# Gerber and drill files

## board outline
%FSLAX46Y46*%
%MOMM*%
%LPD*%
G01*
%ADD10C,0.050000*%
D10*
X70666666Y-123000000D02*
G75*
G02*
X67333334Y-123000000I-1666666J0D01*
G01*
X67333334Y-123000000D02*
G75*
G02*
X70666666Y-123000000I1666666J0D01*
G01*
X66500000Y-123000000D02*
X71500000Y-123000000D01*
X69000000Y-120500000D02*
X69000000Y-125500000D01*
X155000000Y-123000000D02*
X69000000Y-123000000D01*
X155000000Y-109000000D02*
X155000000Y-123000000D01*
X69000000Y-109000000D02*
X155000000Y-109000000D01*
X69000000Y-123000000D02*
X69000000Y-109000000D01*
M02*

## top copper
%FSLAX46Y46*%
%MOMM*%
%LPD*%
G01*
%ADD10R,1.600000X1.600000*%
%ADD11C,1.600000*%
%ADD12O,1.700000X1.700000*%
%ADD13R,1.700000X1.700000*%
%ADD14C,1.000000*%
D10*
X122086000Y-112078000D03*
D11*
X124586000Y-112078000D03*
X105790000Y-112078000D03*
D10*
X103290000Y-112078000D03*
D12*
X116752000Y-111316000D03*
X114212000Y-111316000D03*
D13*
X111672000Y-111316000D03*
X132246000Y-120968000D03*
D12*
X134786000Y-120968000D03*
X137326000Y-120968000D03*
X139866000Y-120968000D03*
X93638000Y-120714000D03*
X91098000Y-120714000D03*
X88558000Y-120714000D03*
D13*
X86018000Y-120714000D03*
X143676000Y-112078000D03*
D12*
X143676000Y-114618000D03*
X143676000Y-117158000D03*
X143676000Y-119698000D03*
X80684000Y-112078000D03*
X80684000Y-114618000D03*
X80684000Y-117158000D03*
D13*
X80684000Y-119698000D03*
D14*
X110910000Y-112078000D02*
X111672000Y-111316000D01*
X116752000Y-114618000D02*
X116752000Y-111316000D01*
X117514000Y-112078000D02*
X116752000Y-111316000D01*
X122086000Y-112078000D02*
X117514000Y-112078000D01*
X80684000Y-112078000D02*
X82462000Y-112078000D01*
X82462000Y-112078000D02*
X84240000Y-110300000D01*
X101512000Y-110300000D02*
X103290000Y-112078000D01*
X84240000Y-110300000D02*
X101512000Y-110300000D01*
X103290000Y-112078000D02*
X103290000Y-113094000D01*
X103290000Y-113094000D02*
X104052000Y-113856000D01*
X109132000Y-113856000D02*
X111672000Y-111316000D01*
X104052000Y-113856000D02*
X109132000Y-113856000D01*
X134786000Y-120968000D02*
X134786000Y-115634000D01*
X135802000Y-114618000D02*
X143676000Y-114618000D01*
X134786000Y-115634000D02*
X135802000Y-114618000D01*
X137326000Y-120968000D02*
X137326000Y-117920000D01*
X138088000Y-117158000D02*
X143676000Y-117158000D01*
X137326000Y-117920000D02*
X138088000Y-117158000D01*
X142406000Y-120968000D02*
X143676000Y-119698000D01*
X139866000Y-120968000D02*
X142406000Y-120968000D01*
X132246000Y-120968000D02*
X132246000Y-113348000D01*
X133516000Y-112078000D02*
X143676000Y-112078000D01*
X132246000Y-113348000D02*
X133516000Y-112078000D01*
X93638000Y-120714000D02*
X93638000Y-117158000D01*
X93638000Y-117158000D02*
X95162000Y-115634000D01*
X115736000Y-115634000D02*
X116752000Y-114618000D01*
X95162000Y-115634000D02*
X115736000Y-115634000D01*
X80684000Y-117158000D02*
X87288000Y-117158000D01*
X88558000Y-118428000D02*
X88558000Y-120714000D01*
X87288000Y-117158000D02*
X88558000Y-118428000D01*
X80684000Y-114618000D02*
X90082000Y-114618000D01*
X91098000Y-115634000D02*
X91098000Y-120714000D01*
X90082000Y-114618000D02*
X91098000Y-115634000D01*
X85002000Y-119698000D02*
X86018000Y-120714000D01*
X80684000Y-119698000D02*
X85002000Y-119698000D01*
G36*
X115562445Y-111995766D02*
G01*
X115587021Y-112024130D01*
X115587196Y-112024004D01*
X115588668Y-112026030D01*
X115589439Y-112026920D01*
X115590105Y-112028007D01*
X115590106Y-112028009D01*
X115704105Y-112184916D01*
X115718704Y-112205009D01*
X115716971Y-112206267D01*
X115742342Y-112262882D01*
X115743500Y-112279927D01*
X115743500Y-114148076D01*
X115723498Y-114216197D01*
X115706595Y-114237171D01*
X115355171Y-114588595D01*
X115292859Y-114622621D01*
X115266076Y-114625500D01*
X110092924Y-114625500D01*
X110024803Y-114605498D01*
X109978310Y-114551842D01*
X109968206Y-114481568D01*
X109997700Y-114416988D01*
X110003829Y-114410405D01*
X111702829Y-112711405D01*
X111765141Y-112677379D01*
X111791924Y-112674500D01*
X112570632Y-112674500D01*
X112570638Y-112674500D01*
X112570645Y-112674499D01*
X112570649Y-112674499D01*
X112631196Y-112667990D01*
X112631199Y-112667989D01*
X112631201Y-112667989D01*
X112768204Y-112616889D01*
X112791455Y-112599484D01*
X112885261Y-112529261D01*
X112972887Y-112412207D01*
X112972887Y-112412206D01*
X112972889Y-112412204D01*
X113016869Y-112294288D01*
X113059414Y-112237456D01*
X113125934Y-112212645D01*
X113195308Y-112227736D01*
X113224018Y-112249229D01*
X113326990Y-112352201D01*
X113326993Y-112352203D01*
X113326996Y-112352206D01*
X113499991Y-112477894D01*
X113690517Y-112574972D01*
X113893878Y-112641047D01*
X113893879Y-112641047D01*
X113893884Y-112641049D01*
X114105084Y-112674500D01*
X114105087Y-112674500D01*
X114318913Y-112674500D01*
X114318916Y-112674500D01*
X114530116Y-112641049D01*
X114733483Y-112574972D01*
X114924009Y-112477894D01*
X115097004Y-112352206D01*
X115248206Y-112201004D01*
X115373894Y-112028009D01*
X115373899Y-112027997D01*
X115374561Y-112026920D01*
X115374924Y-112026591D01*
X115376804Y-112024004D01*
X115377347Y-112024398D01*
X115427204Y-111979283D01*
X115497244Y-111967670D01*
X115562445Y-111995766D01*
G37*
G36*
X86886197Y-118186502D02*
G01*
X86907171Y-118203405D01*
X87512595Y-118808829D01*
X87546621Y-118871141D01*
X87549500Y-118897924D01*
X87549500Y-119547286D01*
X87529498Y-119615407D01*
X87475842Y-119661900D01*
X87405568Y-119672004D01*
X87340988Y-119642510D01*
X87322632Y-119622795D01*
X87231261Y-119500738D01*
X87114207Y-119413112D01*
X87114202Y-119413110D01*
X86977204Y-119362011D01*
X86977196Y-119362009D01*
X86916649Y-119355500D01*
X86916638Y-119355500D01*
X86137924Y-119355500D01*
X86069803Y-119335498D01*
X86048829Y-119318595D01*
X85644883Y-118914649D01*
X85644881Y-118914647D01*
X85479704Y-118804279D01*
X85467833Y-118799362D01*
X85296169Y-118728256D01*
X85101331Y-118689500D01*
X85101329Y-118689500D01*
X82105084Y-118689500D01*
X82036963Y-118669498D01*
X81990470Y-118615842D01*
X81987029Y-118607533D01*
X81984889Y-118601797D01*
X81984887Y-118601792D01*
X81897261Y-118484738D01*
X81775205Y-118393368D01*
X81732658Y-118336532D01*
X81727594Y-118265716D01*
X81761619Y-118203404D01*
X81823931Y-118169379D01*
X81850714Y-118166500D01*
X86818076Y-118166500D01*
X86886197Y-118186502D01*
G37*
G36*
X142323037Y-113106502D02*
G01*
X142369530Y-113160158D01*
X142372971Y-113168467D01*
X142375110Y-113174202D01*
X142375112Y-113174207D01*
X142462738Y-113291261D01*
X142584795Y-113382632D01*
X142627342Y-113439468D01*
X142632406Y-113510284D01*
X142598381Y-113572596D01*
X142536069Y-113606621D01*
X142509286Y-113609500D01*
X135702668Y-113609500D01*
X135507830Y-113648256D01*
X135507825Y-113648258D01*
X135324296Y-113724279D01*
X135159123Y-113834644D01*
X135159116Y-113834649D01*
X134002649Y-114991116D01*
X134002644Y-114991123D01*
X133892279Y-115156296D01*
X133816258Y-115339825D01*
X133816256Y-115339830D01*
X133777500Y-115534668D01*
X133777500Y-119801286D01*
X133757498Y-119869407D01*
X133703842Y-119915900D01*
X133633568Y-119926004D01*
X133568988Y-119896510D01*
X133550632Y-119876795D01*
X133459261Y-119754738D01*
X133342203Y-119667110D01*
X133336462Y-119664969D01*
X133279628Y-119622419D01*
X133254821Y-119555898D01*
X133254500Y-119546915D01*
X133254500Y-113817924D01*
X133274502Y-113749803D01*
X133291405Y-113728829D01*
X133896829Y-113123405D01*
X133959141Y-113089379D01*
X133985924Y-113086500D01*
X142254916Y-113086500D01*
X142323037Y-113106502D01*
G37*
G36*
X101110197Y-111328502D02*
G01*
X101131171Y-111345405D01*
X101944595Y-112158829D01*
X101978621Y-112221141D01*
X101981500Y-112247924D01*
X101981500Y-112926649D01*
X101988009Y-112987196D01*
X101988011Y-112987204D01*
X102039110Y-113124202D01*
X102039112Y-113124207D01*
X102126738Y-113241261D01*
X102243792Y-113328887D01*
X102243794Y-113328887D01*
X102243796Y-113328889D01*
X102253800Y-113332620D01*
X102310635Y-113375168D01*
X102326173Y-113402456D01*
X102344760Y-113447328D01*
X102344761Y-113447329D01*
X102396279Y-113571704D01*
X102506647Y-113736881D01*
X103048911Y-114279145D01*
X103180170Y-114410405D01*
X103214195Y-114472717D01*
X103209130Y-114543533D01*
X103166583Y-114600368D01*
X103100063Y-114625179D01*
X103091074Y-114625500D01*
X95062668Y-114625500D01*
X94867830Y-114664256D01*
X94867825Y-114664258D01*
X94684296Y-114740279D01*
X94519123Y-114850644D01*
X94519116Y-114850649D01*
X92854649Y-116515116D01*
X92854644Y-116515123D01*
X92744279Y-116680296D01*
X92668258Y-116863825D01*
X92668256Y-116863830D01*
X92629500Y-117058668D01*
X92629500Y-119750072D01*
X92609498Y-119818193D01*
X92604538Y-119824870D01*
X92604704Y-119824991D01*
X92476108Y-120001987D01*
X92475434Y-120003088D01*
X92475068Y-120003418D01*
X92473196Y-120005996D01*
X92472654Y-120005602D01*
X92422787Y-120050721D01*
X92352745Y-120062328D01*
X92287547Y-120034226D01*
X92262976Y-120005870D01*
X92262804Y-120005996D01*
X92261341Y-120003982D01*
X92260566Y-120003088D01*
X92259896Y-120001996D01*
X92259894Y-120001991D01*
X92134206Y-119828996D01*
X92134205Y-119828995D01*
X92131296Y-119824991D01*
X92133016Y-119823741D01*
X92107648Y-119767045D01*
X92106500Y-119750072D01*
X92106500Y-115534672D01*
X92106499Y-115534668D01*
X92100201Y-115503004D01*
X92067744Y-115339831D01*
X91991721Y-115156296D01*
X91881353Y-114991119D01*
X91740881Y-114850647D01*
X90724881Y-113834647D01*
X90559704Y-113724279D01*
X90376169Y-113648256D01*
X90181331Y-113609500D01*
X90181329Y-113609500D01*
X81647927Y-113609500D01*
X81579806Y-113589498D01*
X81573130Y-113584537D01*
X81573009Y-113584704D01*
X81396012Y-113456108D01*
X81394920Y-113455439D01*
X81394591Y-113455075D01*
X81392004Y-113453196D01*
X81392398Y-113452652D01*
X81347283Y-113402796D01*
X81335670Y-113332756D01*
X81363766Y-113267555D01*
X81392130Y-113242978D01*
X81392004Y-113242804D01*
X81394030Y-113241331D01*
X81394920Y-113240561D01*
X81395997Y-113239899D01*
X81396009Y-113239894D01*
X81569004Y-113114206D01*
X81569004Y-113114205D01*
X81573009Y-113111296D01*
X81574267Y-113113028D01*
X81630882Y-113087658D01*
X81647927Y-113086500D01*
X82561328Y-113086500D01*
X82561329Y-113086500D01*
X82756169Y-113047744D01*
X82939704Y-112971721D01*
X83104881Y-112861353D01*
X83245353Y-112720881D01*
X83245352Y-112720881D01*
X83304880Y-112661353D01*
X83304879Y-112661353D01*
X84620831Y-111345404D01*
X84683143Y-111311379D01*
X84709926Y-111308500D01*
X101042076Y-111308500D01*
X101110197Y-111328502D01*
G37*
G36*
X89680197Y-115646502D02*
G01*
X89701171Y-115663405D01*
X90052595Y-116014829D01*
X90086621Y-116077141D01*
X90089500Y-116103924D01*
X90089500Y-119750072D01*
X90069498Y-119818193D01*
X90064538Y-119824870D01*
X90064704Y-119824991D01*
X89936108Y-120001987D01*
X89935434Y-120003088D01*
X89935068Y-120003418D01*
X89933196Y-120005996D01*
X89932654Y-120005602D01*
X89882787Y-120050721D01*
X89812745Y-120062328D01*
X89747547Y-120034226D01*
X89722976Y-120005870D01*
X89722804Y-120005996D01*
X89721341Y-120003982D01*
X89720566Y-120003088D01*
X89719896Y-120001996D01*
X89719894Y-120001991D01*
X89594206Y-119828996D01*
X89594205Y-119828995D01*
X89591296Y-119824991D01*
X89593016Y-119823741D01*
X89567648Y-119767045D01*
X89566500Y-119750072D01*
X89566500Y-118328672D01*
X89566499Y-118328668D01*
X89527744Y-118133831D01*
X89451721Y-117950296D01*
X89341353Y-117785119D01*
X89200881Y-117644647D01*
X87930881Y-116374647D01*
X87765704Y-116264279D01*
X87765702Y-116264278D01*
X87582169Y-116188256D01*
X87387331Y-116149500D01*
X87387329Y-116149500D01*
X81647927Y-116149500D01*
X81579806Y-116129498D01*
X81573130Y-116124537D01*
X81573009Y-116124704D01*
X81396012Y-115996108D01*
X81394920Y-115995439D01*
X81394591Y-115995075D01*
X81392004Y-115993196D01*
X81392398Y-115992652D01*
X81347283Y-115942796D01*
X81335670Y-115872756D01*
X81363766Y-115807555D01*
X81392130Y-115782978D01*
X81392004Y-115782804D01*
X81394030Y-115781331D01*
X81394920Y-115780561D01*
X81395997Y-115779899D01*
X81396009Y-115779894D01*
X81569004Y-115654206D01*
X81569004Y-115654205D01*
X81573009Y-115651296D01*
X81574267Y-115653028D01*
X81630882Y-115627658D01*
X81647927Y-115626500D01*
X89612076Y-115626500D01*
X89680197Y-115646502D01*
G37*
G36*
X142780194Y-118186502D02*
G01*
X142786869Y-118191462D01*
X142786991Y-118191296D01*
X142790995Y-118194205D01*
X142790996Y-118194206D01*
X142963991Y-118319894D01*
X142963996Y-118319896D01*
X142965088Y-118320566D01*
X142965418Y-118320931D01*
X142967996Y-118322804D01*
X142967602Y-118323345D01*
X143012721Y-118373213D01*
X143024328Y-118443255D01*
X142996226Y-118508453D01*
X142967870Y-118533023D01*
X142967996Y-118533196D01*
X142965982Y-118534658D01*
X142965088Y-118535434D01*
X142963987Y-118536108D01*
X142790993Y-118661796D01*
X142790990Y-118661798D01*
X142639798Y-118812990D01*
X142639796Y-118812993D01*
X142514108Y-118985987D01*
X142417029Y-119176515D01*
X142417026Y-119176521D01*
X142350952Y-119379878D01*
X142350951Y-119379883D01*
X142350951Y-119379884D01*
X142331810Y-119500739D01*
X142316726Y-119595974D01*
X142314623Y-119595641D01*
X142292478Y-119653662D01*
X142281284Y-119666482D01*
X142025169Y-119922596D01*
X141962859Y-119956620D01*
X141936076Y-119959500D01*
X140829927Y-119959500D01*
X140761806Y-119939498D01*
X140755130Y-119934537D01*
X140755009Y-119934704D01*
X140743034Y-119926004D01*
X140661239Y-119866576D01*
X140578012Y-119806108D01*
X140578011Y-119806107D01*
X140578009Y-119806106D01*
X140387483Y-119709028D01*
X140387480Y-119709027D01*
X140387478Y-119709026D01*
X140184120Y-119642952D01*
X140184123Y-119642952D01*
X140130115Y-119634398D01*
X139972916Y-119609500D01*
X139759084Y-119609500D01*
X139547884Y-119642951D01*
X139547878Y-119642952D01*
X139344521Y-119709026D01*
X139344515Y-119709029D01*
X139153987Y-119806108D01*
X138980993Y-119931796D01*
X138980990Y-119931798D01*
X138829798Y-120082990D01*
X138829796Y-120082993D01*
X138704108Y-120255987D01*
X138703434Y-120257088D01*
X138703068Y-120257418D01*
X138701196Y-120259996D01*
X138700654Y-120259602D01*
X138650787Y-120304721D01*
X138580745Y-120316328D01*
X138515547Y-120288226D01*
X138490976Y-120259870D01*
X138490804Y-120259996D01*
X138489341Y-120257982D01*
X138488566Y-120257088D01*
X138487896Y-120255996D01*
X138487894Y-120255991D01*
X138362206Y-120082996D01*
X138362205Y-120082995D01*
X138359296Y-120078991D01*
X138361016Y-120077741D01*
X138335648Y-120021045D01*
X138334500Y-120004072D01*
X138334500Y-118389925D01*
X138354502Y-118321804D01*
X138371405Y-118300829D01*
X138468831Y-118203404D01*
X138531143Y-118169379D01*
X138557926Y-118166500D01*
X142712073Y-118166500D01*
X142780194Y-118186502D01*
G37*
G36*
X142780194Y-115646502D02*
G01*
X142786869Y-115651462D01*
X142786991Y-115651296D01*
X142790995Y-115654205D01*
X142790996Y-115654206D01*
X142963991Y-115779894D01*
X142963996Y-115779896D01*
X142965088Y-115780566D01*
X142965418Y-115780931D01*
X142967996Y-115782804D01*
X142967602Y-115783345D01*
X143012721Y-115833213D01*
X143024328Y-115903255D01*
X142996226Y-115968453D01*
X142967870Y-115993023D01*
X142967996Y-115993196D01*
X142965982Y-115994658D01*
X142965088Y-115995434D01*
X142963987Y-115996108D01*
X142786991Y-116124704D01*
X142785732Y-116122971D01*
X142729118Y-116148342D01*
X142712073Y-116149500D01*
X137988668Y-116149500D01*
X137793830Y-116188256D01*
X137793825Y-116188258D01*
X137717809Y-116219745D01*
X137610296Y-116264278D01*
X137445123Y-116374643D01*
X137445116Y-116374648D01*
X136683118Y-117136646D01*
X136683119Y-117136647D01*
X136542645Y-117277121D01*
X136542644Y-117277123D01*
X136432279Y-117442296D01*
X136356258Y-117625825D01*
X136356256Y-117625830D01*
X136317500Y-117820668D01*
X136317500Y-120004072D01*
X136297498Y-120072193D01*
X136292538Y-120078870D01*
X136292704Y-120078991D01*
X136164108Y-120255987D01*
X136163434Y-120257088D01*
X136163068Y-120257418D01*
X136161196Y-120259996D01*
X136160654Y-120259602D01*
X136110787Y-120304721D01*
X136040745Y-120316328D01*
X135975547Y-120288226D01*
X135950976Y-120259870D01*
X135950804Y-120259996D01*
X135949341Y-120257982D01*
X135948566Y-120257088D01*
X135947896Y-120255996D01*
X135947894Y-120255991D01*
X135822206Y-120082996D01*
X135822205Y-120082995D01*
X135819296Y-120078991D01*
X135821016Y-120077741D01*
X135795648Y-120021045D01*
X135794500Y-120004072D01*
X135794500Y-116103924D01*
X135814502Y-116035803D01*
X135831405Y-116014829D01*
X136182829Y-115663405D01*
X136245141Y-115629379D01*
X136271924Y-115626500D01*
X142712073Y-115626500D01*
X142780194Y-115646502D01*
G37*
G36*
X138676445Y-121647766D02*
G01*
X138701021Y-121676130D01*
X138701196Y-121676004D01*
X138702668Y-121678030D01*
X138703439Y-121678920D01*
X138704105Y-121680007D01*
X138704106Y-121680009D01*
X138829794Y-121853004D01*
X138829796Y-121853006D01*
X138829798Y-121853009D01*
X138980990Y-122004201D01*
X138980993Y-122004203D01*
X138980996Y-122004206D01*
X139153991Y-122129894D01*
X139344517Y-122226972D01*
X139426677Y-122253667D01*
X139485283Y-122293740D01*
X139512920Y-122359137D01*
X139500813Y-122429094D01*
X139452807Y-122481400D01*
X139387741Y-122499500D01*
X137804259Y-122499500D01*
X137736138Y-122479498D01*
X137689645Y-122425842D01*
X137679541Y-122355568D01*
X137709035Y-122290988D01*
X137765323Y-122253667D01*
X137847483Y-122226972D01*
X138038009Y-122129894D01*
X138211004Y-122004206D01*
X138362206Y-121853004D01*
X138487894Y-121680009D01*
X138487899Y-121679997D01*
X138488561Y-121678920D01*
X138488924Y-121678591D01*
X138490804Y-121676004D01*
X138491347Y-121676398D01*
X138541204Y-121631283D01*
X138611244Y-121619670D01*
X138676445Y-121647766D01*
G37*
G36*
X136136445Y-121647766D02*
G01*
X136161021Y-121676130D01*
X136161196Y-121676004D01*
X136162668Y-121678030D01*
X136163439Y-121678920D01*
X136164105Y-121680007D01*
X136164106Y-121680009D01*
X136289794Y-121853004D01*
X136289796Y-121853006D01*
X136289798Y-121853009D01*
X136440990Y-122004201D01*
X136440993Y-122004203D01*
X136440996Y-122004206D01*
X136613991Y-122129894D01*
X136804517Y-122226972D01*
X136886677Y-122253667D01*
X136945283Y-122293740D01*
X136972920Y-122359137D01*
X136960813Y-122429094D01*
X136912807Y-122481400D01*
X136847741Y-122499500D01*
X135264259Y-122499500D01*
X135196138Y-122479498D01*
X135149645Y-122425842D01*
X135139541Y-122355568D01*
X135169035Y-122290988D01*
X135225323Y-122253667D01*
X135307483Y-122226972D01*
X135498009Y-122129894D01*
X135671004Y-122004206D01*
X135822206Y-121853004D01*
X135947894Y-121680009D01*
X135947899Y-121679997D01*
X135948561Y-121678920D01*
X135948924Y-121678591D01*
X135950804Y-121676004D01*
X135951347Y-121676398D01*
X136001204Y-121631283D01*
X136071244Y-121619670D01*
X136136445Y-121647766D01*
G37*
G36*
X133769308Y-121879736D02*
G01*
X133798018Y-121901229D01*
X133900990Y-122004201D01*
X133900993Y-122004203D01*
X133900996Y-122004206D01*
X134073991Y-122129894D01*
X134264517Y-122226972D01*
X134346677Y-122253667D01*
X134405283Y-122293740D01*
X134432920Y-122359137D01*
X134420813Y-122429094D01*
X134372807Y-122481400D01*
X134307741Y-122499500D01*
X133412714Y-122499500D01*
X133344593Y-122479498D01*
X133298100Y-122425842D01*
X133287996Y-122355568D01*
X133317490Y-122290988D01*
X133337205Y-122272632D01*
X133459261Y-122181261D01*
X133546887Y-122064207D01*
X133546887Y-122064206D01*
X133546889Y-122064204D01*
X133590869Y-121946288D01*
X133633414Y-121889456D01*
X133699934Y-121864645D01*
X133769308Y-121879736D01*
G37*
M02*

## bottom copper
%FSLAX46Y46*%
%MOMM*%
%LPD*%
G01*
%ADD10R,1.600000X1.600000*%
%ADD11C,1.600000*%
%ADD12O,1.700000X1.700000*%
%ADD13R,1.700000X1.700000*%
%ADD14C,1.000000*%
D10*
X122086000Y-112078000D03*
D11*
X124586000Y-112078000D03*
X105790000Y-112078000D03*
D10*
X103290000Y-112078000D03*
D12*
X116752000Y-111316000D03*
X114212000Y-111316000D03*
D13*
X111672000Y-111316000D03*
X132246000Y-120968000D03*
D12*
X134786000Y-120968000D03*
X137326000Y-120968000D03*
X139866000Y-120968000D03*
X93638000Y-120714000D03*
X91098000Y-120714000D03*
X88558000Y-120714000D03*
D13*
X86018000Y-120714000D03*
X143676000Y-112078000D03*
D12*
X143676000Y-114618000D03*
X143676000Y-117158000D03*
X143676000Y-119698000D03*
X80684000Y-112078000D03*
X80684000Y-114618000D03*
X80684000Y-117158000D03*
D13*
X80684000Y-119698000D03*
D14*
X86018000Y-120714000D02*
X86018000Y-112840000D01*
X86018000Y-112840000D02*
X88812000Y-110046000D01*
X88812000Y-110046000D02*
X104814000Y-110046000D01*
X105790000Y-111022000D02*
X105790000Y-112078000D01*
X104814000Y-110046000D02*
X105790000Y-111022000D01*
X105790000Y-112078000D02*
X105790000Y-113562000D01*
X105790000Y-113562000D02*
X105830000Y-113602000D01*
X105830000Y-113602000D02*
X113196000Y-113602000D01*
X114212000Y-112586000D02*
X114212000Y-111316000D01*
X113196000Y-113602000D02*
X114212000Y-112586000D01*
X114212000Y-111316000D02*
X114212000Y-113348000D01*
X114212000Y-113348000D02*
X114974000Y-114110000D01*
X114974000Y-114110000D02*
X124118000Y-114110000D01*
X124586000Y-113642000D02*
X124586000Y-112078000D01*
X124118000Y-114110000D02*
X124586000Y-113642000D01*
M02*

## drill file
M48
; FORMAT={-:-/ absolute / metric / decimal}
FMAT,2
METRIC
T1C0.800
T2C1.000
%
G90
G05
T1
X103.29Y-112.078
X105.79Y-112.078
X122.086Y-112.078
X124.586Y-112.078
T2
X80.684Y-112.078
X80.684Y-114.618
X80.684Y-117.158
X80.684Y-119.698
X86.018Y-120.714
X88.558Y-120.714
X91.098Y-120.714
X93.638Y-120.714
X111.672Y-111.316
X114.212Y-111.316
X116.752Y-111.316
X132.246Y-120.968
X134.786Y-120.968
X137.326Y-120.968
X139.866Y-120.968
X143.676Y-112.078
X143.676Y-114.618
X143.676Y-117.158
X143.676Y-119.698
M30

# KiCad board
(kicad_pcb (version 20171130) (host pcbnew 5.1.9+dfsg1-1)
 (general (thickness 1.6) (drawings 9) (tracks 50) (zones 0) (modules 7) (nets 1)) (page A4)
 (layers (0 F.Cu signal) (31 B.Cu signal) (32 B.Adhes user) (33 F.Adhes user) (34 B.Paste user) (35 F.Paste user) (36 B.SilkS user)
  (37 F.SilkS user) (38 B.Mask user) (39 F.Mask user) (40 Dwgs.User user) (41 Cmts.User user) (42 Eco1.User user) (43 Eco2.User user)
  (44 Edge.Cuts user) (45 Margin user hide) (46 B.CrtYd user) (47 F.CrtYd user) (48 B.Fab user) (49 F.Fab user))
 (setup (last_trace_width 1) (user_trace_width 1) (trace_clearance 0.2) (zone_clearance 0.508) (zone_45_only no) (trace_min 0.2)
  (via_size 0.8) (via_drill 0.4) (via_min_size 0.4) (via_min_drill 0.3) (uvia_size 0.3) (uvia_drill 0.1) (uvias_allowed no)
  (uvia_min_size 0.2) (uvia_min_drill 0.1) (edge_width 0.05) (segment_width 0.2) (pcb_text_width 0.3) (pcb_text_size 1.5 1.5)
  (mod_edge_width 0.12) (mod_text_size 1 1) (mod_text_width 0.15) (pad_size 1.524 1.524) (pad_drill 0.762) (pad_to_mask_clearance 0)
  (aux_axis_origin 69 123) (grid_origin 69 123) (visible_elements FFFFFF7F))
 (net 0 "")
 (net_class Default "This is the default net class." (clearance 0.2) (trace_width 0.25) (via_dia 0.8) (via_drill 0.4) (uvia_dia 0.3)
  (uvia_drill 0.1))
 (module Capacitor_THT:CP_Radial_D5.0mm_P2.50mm (layer F.Cu) (at 122.086 112.078)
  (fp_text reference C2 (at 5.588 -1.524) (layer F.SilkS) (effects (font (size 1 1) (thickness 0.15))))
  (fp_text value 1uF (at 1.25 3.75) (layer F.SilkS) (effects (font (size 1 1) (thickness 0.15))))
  (pad 1 thru_hole rect (at 0 0) (size 1.6 1.6) (drill 0.8) (layers *.Cu *.Mask))
  (pad 2 thru_hole circle (at 2.5 0) (size 1.6 1.6) (drill 0.8) (layers *.Cu *.Mask)))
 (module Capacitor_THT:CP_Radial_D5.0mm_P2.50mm (layer F.Cu) (at 103.29 112.078)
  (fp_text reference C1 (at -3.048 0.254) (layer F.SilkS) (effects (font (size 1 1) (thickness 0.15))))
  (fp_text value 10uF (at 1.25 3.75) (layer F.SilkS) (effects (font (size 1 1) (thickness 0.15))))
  (pad 2 thru_hole circle (at 2.5 0) (size 1.6 1.6) (drill 0.8) (layers *.Cu *.Mask))
  (pad 1 thru_hole rect (at 0 0) (size 1.6 1.6) (drill 0.8) (layers *.Cu *.Mask)))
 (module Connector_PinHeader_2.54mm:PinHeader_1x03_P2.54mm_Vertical (layer F.Cu) (at 111.672 111.316 90)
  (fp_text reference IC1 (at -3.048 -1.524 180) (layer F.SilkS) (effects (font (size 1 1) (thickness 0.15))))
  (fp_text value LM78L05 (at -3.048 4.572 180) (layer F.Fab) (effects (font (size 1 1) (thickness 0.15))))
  (pad 3 thru_hole oval (at 0 5.08 90) (size 1.7 1.7) (drill 1) (layers *.Cu *.Mask))
  (pad 2 thru_hole oval (at 0 2.54 90) (size 1.7 1.7) (drill 1) (layers *.Cu *.Mask))
  (pad 1 thru_hole rect (at 0 0 90) (size 1.7 1.7) (drill 1) (layers *.Cu *.Mask)))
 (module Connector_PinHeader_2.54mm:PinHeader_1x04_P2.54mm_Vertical (layer F.Cu) (at 132.246 120.968 90)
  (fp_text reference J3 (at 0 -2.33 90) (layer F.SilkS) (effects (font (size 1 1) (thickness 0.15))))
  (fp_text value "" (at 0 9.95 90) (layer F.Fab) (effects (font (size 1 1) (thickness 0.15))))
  (pad 1 thru_hole rect (at 0 0 90) (size 1.7 1.7) (drill 1) (layers *.Cu *.Mask))
  (pad 2 thru_hole oval (at 0 2.54 90) (size 1.7 1.7) (drill 1) (layers *.Cu *.Mask))
  (pad 3 thru_hole oval (at 0 5.08 90) (size 1.7 1.7) (drill 1) (layers *.Cu *.Mask))
  (pad 4 thru_hole oval (at 0 7.62 90) (size 1.7 1.7) (drill 1) (layers *.Cu *.Mask)))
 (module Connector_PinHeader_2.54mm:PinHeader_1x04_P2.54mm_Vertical (layer F.Cu) (at 86.018 120.714 90)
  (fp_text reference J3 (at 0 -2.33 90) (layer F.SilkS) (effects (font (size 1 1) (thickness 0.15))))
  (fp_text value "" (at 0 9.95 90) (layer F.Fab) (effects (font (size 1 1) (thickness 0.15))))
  (pad 4 thru_hole oval (at 0 7.62 90) (size 1.7 1.7) (drill 1) (layers *.Cu *.Mask))
  (pad 3 thru_hole oval (at 0 5.08 90) (size 1.7 1.7) (drill 1) (layers *.Cu *.Mask))
  (pad 2 thru_hole oval (at 0 2.54 90) (size 1.7 1.7) (drill 1) (layers *.Cu *.Mask))
  (pad 1 thru_hole rect (at 0 0 90) (size 1.7 1.7) (drill 1) (layers *.Cu *.Mask)))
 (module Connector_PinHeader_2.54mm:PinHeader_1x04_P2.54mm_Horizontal (layer F.Cu) (at 143.676 112.078)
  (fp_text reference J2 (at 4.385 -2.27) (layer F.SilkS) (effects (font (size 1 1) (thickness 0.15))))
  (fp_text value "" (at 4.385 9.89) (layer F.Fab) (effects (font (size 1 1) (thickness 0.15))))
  (pad 1 thru_hole rect (at 0 0) (size 1.7 1.7) (drill 1) (layers *.Cu *.Mask))
  (pad 2 thru_hole oval (at 0 2.54) (size 1.7 1.7) (drill 1) (layers *.Cu *.Mask))
  (pad 3 thru_hole oval (at 0 5.08) (size 1.7 1.7) (drill 1) (layers *.Cu *.Mask))
  (pad 4 thru_hole oval (at 0 7.62) (size 1.7 1.7) (drill 1) (layers *.Cu *.Mask)))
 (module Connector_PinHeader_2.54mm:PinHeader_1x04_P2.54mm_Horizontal (layer F.Cu) (at 80.684 119.698 180)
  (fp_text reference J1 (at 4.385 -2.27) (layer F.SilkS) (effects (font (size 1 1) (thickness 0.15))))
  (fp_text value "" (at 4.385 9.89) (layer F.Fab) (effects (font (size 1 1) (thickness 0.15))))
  (pad 4 thru_hole oval (at 0 7.62 180) (size 1.7 1.7) (drill 1) (layers *.Cu *.Mask))
  (pad 3 thru_hole oval (at 0 5.08 180) (size 1.7 1.7) (drill 1) (layers *.Cu *.Mask))
  (pad 2 thru_hole oval (at 0 2.54 180) (size 1.7 1.7) (drill 1) (layers *.Cu *.Mask))
  (pad 1 thru_hole rect (at 0 0 180) (size 1.7 1.7) (drill 1) (layers *.Cu *.Mask)))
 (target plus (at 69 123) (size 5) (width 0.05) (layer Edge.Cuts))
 (gr_line (start 155 123) (end 69 123) (layer Edge.Cuts) (width 0.05))
 (gr_line (start 155 109) (end 155 123) (layer Edge.Cuts) (width 0.05))
 (gr_line (start 69 109) (end 155 109) (layer Edge.Cuts) (width 0.05))
 (gr_line (start 69 123) (end 69 109) (layer Edge.Cuts) (width 0.05))
 (segment (start 110.91 112.078) (end 111.672 111.316) (width 1) (layer F.Cu) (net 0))
 (segment (start 116.752 114.618) (end 116.752 111.316) (width 1) (layer F.Cu) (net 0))
 (segment (start 117.514 112.078) (end 116.752 111.316) (width 1) (layer F.Cu) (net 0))
 (segment (start 122.086 112.078) (end 117.514 112.078) (width 1) (layer F.Cu) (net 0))
 (segment (start 80.684 112.078) (end 82.462 112.078) (width 1) (layer F.Cu) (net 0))
 (segment (start 82.462 112.078) (end 84.24 110.3) (width 1) (layer F.Cu) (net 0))
 (segment (start 101.512 110.3) (end 103.29 112.078) (width 1) (layer F.Cu) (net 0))
 (segment (start 84.24 110.3) (end 101.512 110.3) (width 1) (layer F.Cu) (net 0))
 (segment (start 103.29 112.078) (end 103.29 113.094) (width 1) (layer F.Cu) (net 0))
 (segment (start 103.29 113.094) (end 104.052 113.856) (width 1) (layer F.Cu) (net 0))
 (segment (start 109.132 113.856) (end 111.672 111.316) (width 1) (layer F.Cu) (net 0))
 (segment (start 104.052 113.856) (end 109.132 113.856) (width 1) (layer F.Cu) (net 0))
 (segment (start 134.786 120.968) (end 134.786 115.634) (width 1) (layer F.Cu) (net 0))
 (segment (start 135.802 114.618) (end 143.676 114.618) (width 1) (layer F.Cu) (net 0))
 (segment (start 134.786 115.634) (end 135.802 114.618) (width 1) (layer F.Cu) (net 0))
 (segment (start 137.326 120.968) (end 137.326 117.92) (width 1) (layer F.Cu) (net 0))
 (segment (start 138.088 117.158) (end 143.676 117.158) (width 1) (layer F.Cu) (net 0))
 (segment (start 137.326 117.92) (end 138.088 117.158) (width 1) (layer F.Cu) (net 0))
 (segment (start 142.406 120.968) (end 143.676 119.698) (width 1) (layer F.Cu) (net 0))
 (segment (start 139.866 120.968) (end 142.406 120.968) (width 1) (layer F.Cu) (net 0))
 (segment (start 132.246 120.968) (end 132.246 113.348) (width 1) (layer F.Cu) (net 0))
 (segment (start 133.516 112.078) (end 143.676 112.078) (width 1) (layer F.Cu) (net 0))
 (segment (start 132.246 113.348) (end 133.516 112.078) (width 1) (layer F.Cu) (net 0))
 (segment (start 93.638 120.714) (end 93.638 117.158) (width 1) (layer F.Cu) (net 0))
 (segment (start 93.638 117.158) (end 95.162 115.634) (width 1) (layer F.Cu) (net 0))
 (segment (start 115.736 115.634) (end 116.752 114.618) (width 1) (layer F.Cu) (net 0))
 (segment (start 95.162 115.634) (end 115.736 115.634) (width 1) (layer F.Cu) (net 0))
 (segment (start 80.684 117.158) (end 87.288 117.158) (width 1) (layer F.Cu) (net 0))
 (segment (start 88.558 118.428) (end 88.558 120.714) (width 1) (layer F.Cu) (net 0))
 (segment (start 87.288 117.158) (end 88.558 118.428) (width 1) (layer F.Cu) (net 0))
 (segment (start 80.684 114.618) (end 90.082 114.618) (width 1) (layer F.Cu) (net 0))
 (segment (start 91.098 115.634) (end 91.098 120.714) (width 1) (layer F.Cu) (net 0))
 (segment (start 90.082 114.618) (end 91.098 115.634) (width 1) (layer F.Cu) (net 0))
 (segment (start 85.002 119.698) (end 86.018 120.714) (width 1) (layer F.Cu) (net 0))
 (segment (start 80.684 119.698) (end 85.002 119.698) (width 1) (layer F.Cu) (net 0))
 (segment (start 86.018 120.714) (end 86.018 112.84) (width 1) (layer B.Cu) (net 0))
 (segment (start 86.018 112.84) (end 88.812 110.046) (width 1) (layer B.Cu) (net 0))
 (segment (start 88.812 110.046) (end 104.814 110.046) (width 1) (layer B.Cu) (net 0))
 (segment (start 105.79 111.022) (end 105.79 112.078) (width 1) (layer B.Cu) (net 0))
 (segment (start 104.814 110.046) (end 105.79 111.022) (width 1) (layer B.Cu) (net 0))
 (segment (start 105.79 112.078) (end 105.79 113.562) (width 1) (layer B.Cu) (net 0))
 (segment (start 105.79 113.562) (end 105.83 113.602) (width 1) (layer B.Cu) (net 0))
 (segment (start 105.83 113.602) (end 113.196 113.602) (width 1) (layer B.Cu) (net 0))
 (segment (start 114.212 112.586) (end 114.212 111.316) (width 1) (layer B.Cu) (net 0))
 (segment (start 113.196 113.602) (end 114.212 112.586) (width 1) (layer B.Cu) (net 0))
 (segment (start 114.212 111.316) (end 114.212 113.348) (width 1) (layer B.Cu) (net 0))
 (segment (start 114.212 113.348) (end 114.974 114.11) (width 1) (layer B.Cu) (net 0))
 (segment (start 114.974 114.11) (end 124.118 114.11) (width 1) (layer B.Cu) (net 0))
 (segment (start 124.586 113.642) (end 124.586 112.078) (width 1) (layer B.Cu) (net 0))
 (segment (start 124.118 114.11) (end 124.586 113.642) (width 1) (layer B.Cu) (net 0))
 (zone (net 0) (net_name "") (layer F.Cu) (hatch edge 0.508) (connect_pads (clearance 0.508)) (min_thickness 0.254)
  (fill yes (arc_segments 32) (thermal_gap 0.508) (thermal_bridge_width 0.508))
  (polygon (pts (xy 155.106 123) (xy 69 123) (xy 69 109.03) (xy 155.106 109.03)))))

